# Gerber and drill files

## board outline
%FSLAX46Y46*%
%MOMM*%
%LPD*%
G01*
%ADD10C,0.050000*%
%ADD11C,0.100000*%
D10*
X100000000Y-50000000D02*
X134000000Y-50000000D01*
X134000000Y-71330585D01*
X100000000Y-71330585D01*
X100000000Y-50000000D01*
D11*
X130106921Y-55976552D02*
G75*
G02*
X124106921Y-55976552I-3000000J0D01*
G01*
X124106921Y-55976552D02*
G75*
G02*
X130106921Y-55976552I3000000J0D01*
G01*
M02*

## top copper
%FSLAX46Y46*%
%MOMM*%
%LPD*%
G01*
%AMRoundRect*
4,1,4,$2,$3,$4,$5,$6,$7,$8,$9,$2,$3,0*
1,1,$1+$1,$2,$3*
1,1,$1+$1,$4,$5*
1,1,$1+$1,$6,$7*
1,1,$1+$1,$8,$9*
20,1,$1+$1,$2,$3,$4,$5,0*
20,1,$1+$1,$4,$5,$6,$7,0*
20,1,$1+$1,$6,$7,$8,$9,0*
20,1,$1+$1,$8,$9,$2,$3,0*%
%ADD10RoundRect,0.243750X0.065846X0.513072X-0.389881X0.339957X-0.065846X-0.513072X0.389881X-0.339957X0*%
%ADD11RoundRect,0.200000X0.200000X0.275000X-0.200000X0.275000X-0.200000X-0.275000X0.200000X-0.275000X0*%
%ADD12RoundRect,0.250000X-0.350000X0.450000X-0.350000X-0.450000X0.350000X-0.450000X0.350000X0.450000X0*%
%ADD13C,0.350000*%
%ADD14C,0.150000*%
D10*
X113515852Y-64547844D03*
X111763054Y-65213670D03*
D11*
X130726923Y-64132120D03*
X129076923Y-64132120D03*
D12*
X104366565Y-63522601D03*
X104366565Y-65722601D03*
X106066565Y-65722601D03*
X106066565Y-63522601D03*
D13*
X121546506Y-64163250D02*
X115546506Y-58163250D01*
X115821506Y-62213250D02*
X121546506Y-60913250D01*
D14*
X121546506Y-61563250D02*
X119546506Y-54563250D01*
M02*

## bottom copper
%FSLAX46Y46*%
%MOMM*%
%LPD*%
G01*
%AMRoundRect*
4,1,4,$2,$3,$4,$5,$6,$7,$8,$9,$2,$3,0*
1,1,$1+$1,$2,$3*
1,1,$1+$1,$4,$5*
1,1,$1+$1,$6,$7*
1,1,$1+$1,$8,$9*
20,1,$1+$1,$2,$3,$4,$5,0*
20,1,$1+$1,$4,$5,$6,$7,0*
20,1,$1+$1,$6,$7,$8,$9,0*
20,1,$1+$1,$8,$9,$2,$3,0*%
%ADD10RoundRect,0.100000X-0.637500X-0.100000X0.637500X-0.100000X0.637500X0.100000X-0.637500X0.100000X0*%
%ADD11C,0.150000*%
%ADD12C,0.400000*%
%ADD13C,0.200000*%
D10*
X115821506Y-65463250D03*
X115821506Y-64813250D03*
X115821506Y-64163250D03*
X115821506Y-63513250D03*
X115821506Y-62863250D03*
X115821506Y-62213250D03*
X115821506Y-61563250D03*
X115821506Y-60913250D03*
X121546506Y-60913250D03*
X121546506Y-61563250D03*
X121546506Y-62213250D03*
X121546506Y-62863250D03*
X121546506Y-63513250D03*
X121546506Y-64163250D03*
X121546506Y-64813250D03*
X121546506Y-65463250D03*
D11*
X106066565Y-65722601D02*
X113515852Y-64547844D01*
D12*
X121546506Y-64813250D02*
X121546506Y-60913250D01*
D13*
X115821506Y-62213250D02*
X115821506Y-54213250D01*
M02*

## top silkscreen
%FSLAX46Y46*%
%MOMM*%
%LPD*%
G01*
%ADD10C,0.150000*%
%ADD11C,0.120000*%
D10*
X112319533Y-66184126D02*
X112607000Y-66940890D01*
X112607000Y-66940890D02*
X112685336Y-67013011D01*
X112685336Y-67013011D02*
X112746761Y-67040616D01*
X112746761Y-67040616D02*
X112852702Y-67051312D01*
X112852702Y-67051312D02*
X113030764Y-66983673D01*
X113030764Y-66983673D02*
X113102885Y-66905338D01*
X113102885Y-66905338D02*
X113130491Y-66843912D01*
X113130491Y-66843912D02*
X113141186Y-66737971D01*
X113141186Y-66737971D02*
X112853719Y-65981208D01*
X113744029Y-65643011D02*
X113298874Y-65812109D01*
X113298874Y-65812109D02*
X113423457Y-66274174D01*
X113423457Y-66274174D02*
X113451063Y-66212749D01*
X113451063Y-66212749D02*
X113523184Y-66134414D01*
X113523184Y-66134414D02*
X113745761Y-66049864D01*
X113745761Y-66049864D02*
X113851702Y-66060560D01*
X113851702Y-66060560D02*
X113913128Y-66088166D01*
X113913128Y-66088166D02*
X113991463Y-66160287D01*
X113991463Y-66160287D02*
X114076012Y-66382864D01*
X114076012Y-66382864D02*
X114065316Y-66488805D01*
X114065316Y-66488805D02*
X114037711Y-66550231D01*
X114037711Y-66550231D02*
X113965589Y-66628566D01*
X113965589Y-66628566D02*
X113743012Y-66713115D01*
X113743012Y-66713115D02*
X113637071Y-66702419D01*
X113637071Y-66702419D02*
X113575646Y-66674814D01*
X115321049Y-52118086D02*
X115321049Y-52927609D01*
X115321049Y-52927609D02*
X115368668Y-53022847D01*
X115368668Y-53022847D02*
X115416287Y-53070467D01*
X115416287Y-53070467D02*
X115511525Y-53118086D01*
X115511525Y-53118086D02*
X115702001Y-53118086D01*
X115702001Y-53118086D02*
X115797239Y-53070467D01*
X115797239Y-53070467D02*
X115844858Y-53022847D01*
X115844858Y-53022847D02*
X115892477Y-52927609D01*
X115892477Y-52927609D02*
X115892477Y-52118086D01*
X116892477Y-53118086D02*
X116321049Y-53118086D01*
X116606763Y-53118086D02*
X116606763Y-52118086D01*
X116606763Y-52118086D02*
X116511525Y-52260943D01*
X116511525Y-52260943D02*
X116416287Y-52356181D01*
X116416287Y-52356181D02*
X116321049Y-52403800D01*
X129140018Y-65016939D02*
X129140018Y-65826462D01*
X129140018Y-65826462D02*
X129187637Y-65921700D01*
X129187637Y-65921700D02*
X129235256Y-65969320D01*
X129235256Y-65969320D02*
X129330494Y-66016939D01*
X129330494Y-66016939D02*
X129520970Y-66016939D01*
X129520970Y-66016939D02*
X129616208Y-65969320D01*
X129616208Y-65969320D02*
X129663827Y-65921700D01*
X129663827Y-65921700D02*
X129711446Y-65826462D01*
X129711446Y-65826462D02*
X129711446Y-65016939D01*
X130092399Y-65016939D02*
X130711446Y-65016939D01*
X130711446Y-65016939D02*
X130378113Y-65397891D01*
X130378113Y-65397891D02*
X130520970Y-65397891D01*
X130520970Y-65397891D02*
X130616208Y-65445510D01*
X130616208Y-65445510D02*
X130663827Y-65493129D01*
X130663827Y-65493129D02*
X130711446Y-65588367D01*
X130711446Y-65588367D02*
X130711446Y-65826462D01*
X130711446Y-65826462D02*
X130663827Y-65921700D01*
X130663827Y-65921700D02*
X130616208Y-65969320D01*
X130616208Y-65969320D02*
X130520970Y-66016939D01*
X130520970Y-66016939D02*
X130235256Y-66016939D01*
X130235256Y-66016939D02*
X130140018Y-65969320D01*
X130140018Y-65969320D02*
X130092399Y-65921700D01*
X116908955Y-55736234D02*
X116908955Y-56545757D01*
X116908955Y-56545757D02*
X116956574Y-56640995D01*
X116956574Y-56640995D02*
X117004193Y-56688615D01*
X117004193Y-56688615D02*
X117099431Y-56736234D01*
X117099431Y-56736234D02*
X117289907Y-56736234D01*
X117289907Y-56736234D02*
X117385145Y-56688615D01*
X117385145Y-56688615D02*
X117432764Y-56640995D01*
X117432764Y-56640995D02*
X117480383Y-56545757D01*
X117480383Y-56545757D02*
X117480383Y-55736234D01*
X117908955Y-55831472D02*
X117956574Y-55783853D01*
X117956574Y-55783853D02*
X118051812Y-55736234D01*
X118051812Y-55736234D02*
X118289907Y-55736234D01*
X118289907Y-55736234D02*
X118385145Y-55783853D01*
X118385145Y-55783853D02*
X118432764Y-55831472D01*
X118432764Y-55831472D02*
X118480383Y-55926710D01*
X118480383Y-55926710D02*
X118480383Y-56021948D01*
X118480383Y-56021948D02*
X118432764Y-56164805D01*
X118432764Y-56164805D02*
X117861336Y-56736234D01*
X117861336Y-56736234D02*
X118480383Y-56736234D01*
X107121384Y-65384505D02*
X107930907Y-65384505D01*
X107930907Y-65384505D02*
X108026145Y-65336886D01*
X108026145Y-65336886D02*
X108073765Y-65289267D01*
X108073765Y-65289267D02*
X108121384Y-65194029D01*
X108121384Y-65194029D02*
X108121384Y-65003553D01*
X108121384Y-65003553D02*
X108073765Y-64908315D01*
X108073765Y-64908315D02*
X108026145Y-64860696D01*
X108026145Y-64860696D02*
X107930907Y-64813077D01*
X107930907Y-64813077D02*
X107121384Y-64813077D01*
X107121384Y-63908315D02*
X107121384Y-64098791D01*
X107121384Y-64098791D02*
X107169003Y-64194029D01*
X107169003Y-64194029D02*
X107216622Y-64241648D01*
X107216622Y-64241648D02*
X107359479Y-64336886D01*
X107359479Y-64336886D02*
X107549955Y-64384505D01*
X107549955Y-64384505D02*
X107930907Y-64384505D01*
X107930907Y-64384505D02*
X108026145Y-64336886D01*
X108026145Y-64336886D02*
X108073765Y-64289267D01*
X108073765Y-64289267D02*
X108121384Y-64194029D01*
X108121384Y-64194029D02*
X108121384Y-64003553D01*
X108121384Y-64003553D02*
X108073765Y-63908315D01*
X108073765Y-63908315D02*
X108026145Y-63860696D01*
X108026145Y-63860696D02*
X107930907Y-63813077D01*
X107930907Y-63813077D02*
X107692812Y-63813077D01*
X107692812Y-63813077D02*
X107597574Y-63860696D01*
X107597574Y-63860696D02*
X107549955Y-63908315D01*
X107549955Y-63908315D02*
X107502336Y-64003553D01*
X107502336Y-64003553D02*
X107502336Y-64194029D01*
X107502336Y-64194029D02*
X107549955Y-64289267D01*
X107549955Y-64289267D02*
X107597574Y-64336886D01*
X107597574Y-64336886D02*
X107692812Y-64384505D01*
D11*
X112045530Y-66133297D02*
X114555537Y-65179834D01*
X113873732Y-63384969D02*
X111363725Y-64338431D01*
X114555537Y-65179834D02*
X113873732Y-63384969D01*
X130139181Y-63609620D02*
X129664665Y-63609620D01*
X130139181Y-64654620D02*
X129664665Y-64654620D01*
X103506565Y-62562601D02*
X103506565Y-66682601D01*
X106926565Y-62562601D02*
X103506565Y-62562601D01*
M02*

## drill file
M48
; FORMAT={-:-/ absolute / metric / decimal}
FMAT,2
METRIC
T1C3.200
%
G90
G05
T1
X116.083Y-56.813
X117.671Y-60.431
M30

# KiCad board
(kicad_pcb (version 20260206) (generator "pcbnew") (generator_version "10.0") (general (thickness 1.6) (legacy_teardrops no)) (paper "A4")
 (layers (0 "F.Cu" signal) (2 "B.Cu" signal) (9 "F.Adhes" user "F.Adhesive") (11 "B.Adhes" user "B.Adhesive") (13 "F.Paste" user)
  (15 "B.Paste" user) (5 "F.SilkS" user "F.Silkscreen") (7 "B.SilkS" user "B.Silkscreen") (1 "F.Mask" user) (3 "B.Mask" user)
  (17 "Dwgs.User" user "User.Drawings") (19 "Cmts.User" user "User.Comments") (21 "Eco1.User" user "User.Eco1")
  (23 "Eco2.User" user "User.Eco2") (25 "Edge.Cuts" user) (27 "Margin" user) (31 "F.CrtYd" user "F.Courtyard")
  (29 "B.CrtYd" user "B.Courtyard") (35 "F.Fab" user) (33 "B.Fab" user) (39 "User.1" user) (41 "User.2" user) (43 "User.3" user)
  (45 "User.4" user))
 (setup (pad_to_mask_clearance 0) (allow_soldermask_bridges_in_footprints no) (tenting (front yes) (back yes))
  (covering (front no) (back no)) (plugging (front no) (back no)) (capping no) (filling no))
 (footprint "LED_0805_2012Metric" (layer "F.Cu") (at 112.639453 64.880757 -159.2)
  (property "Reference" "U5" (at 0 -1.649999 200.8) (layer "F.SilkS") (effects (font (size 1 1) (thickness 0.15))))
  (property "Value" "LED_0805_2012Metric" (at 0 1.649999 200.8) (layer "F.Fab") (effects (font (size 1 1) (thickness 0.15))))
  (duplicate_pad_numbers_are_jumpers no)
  (fp_line (start 1 -0.96) (end -1.685 -0.96) (stroke (width 0.12) (type solid)) (layer "F.SilkS"))
  (fp_line (start -1.685 0.96) (end 1 0.96) (stroke (width 0.12) (type solid)) (layer "F.SilkS"))
  (fp_line (start -1.685 -0.96) (end -1.685 0.96) (stroke (width 0.12) (type solid)) (layer "F.SilkS"))
  (pad "1" smd roundrect (at -0.9375 0 200.8) (size 0.975 1.4) (layers "F.Cu" "F.Mask" "F.Paste") (roundrect_rratio 0.25) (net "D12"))
  (pad "2" smd roundrect (at 0.9375 0 200.8) (size 0.975 1.4) (layers "F.Cu" "F.Mask" "F.Paste") (roundrect_rratio 0.25) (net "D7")))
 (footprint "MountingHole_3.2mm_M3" (layer "F.Cu") (at 116.082954 56.813267)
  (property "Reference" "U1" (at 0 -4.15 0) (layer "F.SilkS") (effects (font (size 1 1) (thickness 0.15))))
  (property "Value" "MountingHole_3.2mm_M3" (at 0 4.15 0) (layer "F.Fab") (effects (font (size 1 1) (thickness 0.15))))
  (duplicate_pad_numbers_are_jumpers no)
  (pad "" np_thru_hole circle (at 0 0) (size 3.2 3.2) (drill 3.2) (layers "*.Cu" "*.Mask")))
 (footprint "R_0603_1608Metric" (layer "F.Cu") (at 129.901923 64.13212 180)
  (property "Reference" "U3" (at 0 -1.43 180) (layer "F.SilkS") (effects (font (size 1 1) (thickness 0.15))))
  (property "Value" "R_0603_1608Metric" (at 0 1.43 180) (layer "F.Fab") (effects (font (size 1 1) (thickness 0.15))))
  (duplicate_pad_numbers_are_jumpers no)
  (fp_line (start -0.237258 0.5225) (end 0.237258 0.5225) (stroke (width 0.12) (type solid)) (layer "F.SilkS"))
  (fp_line (start -0.237258 -0.5225) (end 0.237258 -0.5225) (stroke (width 0.12) (type solid)) (layer "F.SilkS"))
  (pad "1" smd roundrect (at -0.825 0 180) (size 0.8 0.95) (layers "F.Cu" "F.Mask" "F.Paste") (roundrect_rratio 0.25) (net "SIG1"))
  (pad "2" smd roundrect (at 0.825 0 180) (size 0.8 0.95) (layers "F.Cu" "F.Mask" "F.Paste") (roundrect_rratio 0.25)))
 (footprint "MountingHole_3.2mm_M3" (layer "F.Cu") (at 117.67086 60.431415)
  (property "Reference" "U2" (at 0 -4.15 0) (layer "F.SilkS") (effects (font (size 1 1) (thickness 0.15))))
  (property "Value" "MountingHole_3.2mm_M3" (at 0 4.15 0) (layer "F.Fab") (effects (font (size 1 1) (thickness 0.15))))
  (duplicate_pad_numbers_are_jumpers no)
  (pad "" np_thru_hole circle (at 0 0) (size 3.2 3.2) (drill 3.2) (layers "*.Cu" "*.Mask")))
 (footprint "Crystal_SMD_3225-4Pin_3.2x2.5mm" (layer "F.Cu") (at 105.216565 64.622601 -90)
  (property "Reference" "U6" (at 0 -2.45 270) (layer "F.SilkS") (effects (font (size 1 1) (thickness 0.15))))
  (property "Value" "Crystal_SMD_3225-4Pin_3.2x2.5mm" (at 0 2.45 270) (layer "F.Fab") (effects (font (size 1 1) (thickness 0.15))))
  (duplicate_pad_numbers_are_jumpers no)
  (fp_line (start -2.06 1.71) (end 2.06 1.71) (stroke (width 0.12) (type solid)) (layer "F.SilkS"))
  (fp_line (start -2.06 -1.71) (end -2.06 1.71) (stroke (width 0.12) (type solid)) (layer "F.SilkS"))
  (pad "1" smd roundrect (at -1.1 0.85 270) (size 1.4 1.2) (layers "F.Cu" "F.Mask" "F.Paste") (roundrect_rratio 0.208333) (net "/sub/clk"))
  (pad "2" smd roundrect (at 1.1 0.85 270) (size 1.4 1.2) (layers "F.Cu" "F.Mask" "F.Paste") (roundrect_rratio 0.208333) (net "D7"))
  (pad "3" smd roundrect (at 1.1 -0.85 270) (size 1.4 1.2) (layers "F.Cu" "F.Mask" "F.Paste") (roundrect_rratio 0.208333) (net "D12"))
  (pad "4" smd roundrect (at -1.1 -0.85 270) (size 1.4 1.2) (layers "F.Cu" "F.Mask" "F.Paste") (roundrect_rratio 0.208333) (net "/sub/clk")))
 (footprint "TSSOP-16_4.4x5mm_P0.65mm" (layer "B.Cu") (at 118.684006 63.18825)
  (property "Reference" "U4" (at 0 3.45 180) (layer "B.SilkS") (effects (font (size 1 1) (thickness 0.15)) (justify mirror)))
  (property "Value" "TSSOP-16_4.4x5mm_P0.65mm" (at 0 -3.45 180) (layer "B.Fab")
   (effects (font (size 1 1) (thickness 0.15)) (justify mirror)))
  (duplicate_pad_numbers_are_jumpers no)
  (pad "1" smd roundrect (at -2.8625 2.275) (size 1.475 0.4) (layers "B.Cu" "B.Mask" "B.Paste") (roundrect_rratio 0.25) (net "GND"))
  (pad "2" smd roundrect (at -2.8625 1.625) (size 1.475 0.4) (layers "B.Cu" "B.Mask" "B.Paste") (roundrect_rratio 0.25) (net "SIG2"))
  (pad "3" smd roundrect (at -2.8625 0.975) (size 1.475 0.4) (layers "B.Cu" "B.Mask" "B.Paste") (roundrect_rratio 0.25) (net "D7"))
  (pad "4" smd roundrect (at -2.8625 0.325) (size 1.475 0.4) (layers "B.Cu" "B.Mask" "B.Paste") (roundrect_rratio 0.25) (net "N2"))
  (pad "5" smd roundrect (at -2.8625 -0.325) (size 1.475 0.4) (layers "B.Cu" "B.Mask" "B.Paste") (roundrect_rratio 0.25) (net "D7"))
  (pad "6" smd roundrect (at -2.8625 -0.975) (size 1.475 0.4) (layers "B.Cu" "B.Mask" "B.Paste") (roundrect_rratio 0.25) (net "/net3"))
  (pad "7" smd roundrect (at -2.8625 -1.625) (size 1.475 0.4) (layers "B.Cu" "B.Mask" "B.Paste") (roundrect_rratio 0.25))
  (pad "8" smd roundrect (at -2.8625 -2.275) (size 1.475 0.4) (layers "B.Cu" "B.Mask" "B.Paste") (roundrect_rratio 0.25) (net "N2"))
  (pad "9" smd roundrect (at 2.8625 -2.275) (size 1.475 0.4) (layers "B.Cu" "B.Mask" "B.Paste") (roundrect_rratio 0.25))
  (pad "10" smd roundrect (at 2.8625 -1.625) (size 1.475 0.4) (layers "B.Cu" "B.Mask" "B.Paste") (roundrect_rratio 0.25) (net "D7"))
  (pad "11" smd roundrect (at 2.8625 -0.975) (size 1.475 0.4) (layers "B.Cu" "B.Mask" "B.Paste") (roundrect_rratio 0.25) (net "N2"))
  (pad "12" smd roundrect (at 2.8625 -0.325) (size 1.475 0.4) (layers "B.Cu" "B.Mask" "B.Paste") (roundrect_rratio 0.25))
  (pad "13" smd roundrect (at 2.8625 0.325) (size 1.475 0.4) (layers "B.Cu" "B.Mask" "B.Paste") (roundrect_rratio 0.25))
  (pad "14" smd roundrect (at 2.8625 0.975) (size 1.475 0.4) (layers "B.Cu" "B.Mask" "B.Paste") (roundrect_rratio 0.25) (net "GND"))
  (pad "15" smd roundrect (at 2.8625 1.625) (size 1.475 0.4) (layers "B.Cu" "B.Mask" "B.Paste") (roundrect_rratio 0.25) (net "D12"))
  (pad "16" smd roundrect (at 2.8625 2.275) (size 1.475 0.4) (layers "B.Cu" "B.Mask" "B.Paste") (roundrect_rratio 0.25)))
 (gr_rect (start 100 50) (end 134 71.330585) (stroke (width 0.05) (type default)) (fill no) (layer "Edge.Cuts"))
 (gr_circle (center 127.106921 55.976552) (end 130.106921 55.976552) (stroke (width 0.1) (type default)) (fill no) (layer "Edge.Cuts"))
 (segment (start 121.546506 64.16325) (end 115.546506 58.16325) (width 0.35) (layer "F.Cu") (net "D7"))
 (segment (start 115.821506 62.21325) (end 121.546506 60.91325) (width 0.35) (layer "F.Cu") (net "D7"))
 (segment (start 121.546506 61.56325) (end 119.546506 54.56325) (width 0.15) (layer "F.Cu") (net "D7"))
 (segment (start 106.066565 65.722601) (end 113.515852 64.547844) (width 0.15) (layer "B.Cu") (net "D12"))
 (segment (start 121.546506 64.81325) (end 121.546506 60.91325) (width 0.4) (layer "B.Cu") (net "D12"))
 (segment (start 115.821506 62.21325) (end 115.821506 54.21325) (width 0.2) (layer "B.Cu") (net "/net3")))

